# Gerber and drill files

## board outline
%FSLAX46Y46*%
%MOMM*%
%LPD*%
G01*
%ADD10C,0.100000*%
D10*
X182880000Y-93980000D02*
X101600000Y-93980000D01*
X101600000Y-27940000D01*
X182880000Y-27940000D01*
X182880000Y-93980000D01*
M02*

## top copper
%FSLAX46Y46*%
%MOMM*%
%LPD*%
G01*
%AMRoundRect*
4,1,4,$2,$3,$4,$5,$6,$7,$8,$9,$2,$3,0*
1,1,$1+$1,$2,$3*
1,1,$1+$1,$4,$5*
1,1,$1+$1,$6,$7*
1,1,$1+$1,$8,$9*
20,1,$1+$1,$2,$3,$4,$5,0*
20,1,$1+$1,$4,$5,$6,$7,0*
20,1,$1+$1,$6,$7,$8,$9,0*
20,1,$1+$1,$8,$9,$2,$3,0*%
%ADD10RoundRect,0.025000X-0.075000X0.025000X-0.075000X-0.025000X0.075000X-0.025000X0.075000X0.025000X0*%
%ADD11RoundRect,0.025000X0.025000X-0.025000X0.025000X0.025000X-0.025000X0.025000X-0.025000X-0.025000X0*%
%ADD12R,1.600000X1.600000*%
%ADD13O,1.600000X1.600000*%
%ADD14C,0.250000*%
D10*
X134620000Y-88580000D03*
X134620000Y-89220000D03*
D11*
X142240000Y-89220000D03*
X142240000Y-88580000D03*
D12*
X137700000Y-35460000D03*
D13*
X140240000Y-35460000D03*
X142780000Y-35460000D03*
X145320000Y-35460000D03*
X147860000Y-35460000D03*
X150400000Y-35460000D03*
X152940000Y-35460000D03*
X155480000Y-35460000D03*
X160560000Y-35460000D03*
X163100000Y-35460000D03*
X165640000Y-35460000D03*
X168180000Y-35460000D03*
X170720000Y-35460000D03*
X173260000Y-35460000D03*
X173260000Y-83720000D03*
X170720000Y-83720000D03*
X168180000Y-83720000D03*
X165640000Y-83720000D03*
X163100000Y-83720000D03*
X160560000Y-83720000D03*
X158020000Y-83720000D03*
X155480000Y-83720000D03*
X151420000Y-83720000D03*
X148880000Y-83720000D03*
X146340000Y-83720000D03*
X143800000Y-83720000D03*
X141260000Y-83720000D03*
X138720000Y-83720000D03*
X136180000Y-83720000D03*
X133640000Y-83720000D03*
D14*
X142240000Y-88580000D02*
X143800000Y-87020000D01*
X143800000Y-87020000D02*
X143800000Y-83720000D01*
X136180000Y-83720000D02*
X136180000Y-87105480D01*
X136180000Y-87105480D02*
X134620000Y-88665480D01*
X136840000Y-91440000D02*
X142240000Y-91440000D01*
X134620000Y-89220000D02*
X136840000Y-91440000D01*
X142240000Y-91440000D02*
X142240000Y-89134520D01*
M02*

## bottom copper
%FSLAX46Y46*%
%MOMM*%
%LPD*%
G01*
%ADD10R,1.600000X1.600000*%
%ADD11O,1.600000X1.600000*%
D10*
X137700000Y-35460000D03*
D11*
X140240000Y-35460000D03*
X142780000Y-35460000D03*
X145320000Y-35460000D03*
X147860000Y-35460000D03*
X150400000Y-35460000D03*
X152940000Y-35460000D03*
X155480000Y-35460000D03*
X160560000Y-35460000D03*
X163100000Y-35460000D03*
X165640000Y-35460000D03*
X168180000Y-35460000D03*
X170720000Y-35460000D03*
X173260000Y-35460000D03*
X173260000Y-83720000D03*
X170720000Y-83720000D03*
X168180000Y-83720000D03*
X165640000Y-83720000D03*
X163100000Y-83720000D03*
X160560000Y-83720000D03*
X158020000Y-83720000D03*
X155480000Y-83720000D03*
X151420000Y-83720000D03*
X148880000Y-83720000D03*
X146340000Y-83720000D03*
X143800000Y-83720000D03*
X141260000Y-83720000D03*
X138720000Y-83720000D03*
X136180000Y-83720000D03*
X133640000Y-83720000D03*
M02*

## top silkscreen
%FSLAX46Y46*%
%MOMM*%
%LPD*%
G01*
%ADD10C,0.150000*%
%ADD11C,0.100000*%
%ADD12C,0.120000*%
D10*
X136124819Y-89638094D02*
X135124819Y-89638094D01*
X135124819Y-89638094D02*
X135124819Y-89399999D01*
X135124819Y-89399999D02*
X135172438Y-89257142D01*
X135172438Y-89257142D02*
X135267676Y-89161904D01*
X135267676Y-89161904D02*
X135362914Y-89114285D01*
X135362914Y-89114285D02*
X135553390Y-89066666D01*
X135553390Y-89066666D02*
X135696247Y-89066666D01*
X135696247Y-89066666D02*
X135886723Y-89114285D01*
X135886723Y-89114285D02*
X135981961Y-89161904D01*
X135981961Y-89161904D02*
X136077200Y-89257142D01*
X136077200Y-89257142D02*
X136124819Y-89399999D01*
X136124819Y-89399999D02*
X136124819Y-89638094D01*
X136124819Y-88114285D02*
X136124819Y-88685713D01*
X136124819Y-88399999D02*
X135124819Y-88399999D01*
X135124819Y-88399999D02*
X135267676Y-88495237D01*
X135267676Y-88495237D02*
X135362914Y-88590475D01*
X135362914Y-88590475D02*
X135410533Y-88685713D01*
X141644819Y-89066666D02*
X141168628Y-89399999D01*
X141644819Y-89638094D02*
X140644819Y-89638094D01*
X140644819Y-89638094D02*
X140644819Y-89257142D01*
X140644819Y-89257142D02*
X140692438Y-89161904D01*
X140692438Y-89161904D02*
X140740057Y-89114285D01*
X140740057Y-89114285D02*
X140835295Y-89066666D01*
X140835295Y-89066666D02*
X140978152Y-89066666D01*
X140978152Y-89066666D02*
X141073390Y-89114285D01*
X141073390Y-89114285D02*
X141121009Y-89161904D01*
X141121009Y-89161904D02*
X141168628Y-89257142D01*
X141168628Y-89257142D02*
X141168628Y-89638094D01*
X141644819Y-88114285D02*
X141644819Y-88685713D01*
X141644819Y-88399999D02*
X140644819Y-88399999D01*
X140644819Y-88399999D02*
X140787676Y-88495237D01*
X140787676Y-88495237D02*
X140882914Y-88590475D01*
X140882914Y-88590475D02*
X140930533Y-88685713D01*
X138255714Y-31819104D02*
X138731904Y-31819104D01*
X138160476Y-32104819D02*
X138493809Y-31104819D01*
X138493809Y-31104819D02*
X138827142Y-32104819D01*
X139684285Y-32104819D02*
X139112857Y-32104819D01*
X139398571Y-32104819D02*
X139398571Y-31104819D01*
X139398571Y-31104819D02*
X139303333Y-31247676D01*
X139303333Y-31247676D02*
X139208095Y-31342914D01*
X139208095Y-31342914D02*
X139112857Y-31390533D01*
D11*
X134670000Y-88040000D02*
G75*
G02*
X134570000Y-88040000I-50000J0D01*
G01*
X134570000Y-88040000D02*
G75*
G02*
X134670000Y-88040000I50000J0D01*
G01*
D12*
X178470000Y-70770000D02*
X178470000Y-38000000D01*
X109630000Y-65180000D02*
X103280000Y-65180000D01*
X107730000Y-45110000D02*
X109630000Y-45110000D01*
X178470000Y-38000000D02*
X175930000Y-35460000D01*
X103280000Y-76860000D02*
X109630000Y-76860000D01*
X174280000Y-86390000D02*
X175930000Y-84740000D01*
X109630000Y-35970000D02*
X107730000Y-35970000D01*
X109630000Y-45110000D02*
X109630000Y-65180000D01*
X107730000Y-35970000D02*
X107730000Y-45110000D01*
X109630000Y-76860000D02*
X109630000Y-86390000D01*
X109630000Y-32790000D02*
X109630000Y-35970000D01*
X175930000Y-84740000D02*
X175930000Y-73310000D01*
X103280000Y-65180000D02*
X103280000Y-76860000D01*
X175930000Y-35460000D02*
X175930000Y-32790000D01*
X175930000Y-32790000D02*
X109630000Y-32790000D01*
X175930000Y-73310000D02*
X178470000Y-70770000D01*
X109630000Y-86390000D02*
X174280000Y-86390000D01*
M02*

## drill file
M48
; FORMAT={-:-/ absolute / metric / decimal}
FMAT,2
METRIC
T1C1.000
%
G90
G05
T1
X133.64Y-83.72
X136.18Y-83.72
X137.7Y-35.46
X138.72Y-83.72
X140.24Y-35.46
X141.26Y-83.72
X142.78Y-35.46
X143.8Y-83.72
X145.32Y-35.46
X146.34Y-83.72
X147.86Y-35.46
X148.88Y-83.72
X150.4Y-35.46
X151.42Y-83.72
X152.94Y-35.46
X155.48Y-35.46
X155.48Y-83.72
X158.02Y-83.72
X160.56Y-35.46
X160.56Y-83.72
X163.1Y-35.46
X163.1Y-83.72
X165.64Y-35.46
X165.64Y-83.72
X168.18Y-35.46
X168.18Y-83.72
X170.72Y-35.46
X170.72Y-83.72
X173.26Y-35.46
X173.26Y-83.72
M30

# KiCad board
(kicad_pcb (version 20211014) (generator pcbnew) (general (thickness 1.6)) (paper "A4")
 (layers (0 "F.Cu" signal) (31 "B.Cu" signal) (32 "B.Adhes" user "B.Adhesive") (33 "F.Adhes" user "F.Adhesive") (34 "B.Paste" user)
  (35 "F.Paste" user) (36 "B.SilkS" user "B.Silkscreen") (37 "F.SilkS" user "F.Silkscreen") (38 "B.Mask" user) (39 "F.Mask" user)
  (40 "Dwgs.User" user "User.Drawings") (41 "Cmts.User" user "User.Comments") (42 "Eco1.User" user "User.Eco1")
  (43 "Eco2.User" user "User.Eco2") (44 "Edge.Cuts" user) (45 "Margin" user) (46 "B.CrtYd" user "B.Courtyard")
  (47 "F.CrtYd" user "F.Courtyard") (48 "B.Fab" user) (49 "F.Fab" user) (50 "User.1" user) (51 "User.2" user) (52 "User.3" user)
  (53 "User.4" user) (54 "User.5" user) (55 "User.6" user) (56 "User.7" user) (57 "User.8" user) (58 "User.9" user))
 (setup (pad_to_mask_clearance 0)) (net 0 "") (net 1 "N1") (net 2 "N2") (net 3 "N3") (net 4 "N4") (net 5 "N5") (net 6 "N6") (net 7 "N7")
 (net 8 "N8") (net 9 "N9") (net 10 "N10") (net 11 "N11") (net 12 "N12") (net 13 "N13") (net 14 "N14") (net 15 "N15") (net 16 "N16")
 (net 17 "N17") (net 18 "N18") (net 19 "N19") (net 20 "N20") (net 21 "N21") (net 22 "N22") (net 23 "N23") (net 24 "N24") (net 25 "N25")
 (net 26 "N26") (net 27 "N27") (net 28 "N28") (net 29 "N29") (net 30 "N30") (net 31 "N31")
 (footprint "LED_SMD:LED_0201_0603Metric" (layer "F.Cu") (at 134.62 88.9 -90)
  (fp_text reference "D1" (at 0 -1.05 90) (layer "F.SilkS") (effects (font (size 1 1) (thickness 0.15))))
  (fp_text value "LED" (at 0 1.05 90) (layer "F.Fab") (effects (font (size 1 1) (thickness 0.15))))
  (fp_circle (center -0.86 0) (end -0.81 0) (layer "F.SilkS") (width 0.1) (fill none))
  (pad "" smd roundrect (at -0.345 0 270) (size 0.318 0.36) (layers "F.Paste") (roundrect_rratio 0.25))
  (pad "" smd roundrect (at 0.345 0 270) (size 0.318 0.36) (layers "F.Paste") (roundrect_rratio 0.25))
  (pad "1" smd roundrect (at -0.32 0 270) (size 0.1 0.2) (layers "F.Cu" "F.Mask") (roundrect_rratio 0.25) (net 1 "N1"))
  (pad "2" smd roundrect (at 0.32 0 270) (size 0.1 0.2) (layers "F.Cu" "F.Mask") (roundrect_rratio 0.25) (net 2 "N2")))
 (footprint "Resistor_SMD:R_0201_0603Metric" (layer "F.Cu") (at 142.24 88.9 90)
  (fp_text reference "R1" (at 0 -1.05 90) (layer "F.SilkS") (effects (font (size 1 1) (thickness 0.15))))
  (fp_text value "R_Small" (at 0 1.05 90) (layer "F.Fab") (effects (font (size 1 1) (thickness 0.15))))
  (pad "" smd roundrect (at 0.345 0 90) (size 0.1 0.2) (layers "F.Paste") (roundrect_rratio 0.25))
  (pad "" smd roundrect (at -0.345 0 90) (size 0.05 0.05) (layers "F.Paste") (roundrect_rratio 0.25))
  (pad "1" smd roundrect (at -0.32 0 90) (size 0.1 0.1) (layers "F.Cu" "F.Mask") (roundrect_rratio 0.25) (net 2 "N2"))
  (pad "2" smd roundrect (at 0.32 0 90) (size 0.1 0.1) (layers "F.Cu" "F.Mask") (roundrect_rratio 0.25) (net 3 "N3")))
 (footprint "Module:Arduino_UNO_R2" (layer "F.Cu") (at 137.7 35.46)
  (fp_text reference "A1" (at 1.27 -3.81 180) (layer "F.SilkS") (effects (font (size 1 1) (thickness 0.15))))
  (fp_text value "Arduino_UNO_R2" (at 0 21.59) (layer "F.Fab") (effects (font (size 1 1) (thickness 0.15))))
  (fp_line (start 40.77 35.31) (end 40.77 2.54) (layer "F.SilkS") (width 0.12))
  (fp_line (start -28.07 29.72) (end -34.42 29.72) (layer "F.SilkS") (width 0.12))
  (fp_line (start -29.97 9.65) (end -28.07 9.65) (layer "F.SilkS") (width 0.12))
  (fp_line (start 40.77 2.54) (end 38.23 0) (layer "F.SilkS") (width 0.12))
  (fp_line (start -34.42 41.4) (end -28.07 41.4) (layer "F.SilkS") (width 0.12))
  (fp_line (start 36.58 50.93) (end 38.23 49.28) (layer "F.SilkS") (width 0.12))
  (fp_line (start -28.07 0.51) (end -29.97 0.51) (layer "F.SilkS") (width 0.12))
  (fp_line (start -28.07 9.65) (end -28.07 29.72) (layer "F.SilkS") (width 0.12))
  (fp_line (start -29.97 0.51) (end -29.97 9.65) (layer "F.SilkS") (width 0.12))
  (fp_line (start -28.07 41.4) (end -28.07 50.93) (layer "F.SilkS") (width 0.12))
  (fp_line (start -28.07 -2.67) (end -28.07 0.51) (layer "F.SilkS") (width 0.12))
  (fp_line (start 38.23 49.28) (end 38.23 37.85) (layer "F.SilkS") (width 0.12))
  (fp_line (start -34.42 29.72) (end -34.42 41.4) (layer "F.SilkS") (width 0.12))
  (fp_line (start 38.23 0) (end 38.23 -2.67) (layer "F.SilkS") (width 0.12))
  (fp_line (start 38.23 -2.67) (end -28.07 -2.67) (layer "F.SilkS") (width 0.12))
  (fp_line (start 38.23 37.85) (end 40.77 35.31) (layer "F.SilkS") (width 0.12))
  (fp_line (start -28.07 50.93) (end 36.58 50.93) (layer "F.SilkS") (width 0.12))
  (pad "1" thru_hole rect (at 0 0 90) (size 1.6 1.6) (drill 1) (layers *.Cu *.Mask) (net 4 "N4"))
  (pad "2" thru_hole oval (at 2.54 0 90) (size 1.6 1.6) (drill 1) (layers *.Cu *.Mask) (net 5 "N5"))
  (pad "3" thru_hole oval (at 5.08 0 90) (size 1.6 1.6) (drill 1) (layers *.Cu *.Mask) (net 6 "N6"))
  (pad "4" thru_hole oval (at 7.62 0 90) (size 1.6 1.6) (drill 1) (layers *.Cu *.Mask) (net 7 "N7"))
  (pad "5" thru_hole oval (at 10.16 0 90) (size 1.6 1.6) (drill 1) (layers *.Cu *.Mask) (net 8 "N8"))
  (pad "6" thru_hole oval (at 12.7 0 90) (size 1.6 1.6) (drill 1) (layers *.Cu *.Mask) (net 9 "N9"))
  (pad "7" thru_hole oval (at 15.24 0 90) (size 1.6 1.6) (drill 1) (layers *.Cu *.Mask) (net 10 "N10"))
  (pad "8" thru_hole oval (at 17.78 0 90) (size 1.6 1.6) (drill 1) (layers *.Cu *.Mask) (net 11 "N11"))
  (pad "9" thru_hole oval (at 22.86 0 90) (size 1.6 1.6) (drill 1) (layers *.Cu *.Mask) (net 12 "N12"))
  (pad "10" thru_hole oval (at 25.4 0 90) (size 1.6 1.6) (drill 1) (layers *.Cu *.Mask) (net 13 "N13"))
  (pad "11" thru_hole oval (at 27.94 0 90) (size 1.6 1.6) (drill 1) (layers *.Cu *.Mask) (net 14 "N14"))
  (pad "12" thru_hole oval (at 30.48 0 90) (size 1.6 1.6) (drill 1) (layers *.Cu *.Mask) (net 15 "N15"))
  (pad "13" thru_hole oval (at 33.02 0 90) (size 1.6 1.6) (drill 1) (layers *.Cu *.Mask) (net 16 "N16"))
  (pad "14" thru_hole oval (at 35.56 0 90) (size 1.6 1.6) (drill 1) (layers *.Cu *.Mask) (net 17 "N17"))
  (pad "15" thru_hole oval (at 35.56 48.26 90) (size 1.6 1.6) (drill 1) (layers *.Cu *.Mask) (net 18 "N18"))
  (pad "16" thru_hole oval (at 33.02 48.26 90) (size 1.6 1.6) (drill 1) (layers *.Cu *.Mask) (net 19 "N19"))
  (pad "17" thru_hole oval (at 30.48 48.26 90) (size 1.6 1.6) (drill 1) (layers *.Cu *.Mask) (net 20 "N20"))
  (pad "18" thru_hole oval (at 27.94 48.26 90) (size 1.6 1.6) (drill 1) (layers *.Cu *.Mask) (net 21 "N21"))
  (pad "19" thru_hole oval (at 25.4 48.26 90) (size 1.6 1.6) (drill 1) (layers *.Cu *.Mask) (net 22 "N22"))
  (pad "20" thru_hole oval (at 22.86 48.26 90) (size 1.6 1.6) (drill 1) (layers *.Cu *.Mask) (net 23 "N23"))
  (pad "21" thru_hole oval (at 20.32 48.26 90) (size 1.6 1.6) (drill 1) (layers *.Cu *.Mask) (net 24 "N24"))
  (pad "22" thru_hole oval (at 17.78 48.26 90) (size 1.6 1.6) (drill 1) (layers *.Cu *.Mask) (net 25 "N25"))
  (pad "23" thru_hole oval (at 13.72 48.26 90) (size 1.6 1.6) (drill 1) (layers *.Cu *.Mask) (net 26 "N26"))
  (pad "24" thru_hole oval (at 11.18 48.26 90) (size 1.6 1.6) (drill 1) (layers *.Cu *.Mask) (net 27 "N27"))
  (pad "25" thru_hole oval (at 8.64 48.26 90) (size 1.6 1.6) (drill 1) (layers *.Cu *.Mask) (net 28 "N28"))
  (pad "26" thru_hole oval (at 6.1 48.26 90) (size 1.6 1.6) (drill 1) (layers *.Cu *.Mask) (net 3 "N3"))
  (pad "27" thru_hole oval (at 3.56 48.26 90) (size 1.6 1.6) (drill 1) (layers *.Cu *.Mask) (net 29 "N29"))
  (pad "28" thru_hole oval (at 1.02 48.26 90) (size 1.6 1.6) (drill 1) (layers *.Cu *.Mask) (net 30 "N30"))
  (pad "29" thru_hole oval (at -1.52 48.26 90) (size 1.6 1.6) (drill 1) (layers *.Cu *.Mask) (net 1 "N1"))
  (pad "30" thru_hole oval (at -4.06 48.26 90) (size 1.6 1.6) (drill 1) (layers *.Cu *.Mask) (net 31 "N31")))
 (gr_poly (pts (xy 182.88 93.98) (xy 101.6 93.98) (xy 101.6 27.94) (xy 182.88 27.94)) (layer "Edge.Cuts") (width 0.1) (fill none))
 (segment (start 142.24 88.58) (end 143.8 87.02) (width 0.25) (layer "F.Cu") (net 3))
 (segment (start 143.8 87.02) (end 143.8 83.72) (width 0.25) (layer "F.Cu") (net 3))
 (segment (start 136.18 83.72) (end 136.18 87.10548) (width 0.25) (layer "F.Cu") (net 1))
 (segment (start 136.18 87.10548) (end 134.62 88.66548) (width 0.25) (layer "F.Cu") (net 1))
 (segment (start 136.84 91.44) (end 142.24 91.44) (width 0.25) (layer "F.Cu") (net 2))
 (segment (start 134.62 89.22) (end 136.84 91.44) (width 0.25) (layer "F.Cu") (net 2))
 (segment (start 142.24 91.44) (end 142.24 89.13452) (width 0.25) (layer "F.Cu") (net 2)))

